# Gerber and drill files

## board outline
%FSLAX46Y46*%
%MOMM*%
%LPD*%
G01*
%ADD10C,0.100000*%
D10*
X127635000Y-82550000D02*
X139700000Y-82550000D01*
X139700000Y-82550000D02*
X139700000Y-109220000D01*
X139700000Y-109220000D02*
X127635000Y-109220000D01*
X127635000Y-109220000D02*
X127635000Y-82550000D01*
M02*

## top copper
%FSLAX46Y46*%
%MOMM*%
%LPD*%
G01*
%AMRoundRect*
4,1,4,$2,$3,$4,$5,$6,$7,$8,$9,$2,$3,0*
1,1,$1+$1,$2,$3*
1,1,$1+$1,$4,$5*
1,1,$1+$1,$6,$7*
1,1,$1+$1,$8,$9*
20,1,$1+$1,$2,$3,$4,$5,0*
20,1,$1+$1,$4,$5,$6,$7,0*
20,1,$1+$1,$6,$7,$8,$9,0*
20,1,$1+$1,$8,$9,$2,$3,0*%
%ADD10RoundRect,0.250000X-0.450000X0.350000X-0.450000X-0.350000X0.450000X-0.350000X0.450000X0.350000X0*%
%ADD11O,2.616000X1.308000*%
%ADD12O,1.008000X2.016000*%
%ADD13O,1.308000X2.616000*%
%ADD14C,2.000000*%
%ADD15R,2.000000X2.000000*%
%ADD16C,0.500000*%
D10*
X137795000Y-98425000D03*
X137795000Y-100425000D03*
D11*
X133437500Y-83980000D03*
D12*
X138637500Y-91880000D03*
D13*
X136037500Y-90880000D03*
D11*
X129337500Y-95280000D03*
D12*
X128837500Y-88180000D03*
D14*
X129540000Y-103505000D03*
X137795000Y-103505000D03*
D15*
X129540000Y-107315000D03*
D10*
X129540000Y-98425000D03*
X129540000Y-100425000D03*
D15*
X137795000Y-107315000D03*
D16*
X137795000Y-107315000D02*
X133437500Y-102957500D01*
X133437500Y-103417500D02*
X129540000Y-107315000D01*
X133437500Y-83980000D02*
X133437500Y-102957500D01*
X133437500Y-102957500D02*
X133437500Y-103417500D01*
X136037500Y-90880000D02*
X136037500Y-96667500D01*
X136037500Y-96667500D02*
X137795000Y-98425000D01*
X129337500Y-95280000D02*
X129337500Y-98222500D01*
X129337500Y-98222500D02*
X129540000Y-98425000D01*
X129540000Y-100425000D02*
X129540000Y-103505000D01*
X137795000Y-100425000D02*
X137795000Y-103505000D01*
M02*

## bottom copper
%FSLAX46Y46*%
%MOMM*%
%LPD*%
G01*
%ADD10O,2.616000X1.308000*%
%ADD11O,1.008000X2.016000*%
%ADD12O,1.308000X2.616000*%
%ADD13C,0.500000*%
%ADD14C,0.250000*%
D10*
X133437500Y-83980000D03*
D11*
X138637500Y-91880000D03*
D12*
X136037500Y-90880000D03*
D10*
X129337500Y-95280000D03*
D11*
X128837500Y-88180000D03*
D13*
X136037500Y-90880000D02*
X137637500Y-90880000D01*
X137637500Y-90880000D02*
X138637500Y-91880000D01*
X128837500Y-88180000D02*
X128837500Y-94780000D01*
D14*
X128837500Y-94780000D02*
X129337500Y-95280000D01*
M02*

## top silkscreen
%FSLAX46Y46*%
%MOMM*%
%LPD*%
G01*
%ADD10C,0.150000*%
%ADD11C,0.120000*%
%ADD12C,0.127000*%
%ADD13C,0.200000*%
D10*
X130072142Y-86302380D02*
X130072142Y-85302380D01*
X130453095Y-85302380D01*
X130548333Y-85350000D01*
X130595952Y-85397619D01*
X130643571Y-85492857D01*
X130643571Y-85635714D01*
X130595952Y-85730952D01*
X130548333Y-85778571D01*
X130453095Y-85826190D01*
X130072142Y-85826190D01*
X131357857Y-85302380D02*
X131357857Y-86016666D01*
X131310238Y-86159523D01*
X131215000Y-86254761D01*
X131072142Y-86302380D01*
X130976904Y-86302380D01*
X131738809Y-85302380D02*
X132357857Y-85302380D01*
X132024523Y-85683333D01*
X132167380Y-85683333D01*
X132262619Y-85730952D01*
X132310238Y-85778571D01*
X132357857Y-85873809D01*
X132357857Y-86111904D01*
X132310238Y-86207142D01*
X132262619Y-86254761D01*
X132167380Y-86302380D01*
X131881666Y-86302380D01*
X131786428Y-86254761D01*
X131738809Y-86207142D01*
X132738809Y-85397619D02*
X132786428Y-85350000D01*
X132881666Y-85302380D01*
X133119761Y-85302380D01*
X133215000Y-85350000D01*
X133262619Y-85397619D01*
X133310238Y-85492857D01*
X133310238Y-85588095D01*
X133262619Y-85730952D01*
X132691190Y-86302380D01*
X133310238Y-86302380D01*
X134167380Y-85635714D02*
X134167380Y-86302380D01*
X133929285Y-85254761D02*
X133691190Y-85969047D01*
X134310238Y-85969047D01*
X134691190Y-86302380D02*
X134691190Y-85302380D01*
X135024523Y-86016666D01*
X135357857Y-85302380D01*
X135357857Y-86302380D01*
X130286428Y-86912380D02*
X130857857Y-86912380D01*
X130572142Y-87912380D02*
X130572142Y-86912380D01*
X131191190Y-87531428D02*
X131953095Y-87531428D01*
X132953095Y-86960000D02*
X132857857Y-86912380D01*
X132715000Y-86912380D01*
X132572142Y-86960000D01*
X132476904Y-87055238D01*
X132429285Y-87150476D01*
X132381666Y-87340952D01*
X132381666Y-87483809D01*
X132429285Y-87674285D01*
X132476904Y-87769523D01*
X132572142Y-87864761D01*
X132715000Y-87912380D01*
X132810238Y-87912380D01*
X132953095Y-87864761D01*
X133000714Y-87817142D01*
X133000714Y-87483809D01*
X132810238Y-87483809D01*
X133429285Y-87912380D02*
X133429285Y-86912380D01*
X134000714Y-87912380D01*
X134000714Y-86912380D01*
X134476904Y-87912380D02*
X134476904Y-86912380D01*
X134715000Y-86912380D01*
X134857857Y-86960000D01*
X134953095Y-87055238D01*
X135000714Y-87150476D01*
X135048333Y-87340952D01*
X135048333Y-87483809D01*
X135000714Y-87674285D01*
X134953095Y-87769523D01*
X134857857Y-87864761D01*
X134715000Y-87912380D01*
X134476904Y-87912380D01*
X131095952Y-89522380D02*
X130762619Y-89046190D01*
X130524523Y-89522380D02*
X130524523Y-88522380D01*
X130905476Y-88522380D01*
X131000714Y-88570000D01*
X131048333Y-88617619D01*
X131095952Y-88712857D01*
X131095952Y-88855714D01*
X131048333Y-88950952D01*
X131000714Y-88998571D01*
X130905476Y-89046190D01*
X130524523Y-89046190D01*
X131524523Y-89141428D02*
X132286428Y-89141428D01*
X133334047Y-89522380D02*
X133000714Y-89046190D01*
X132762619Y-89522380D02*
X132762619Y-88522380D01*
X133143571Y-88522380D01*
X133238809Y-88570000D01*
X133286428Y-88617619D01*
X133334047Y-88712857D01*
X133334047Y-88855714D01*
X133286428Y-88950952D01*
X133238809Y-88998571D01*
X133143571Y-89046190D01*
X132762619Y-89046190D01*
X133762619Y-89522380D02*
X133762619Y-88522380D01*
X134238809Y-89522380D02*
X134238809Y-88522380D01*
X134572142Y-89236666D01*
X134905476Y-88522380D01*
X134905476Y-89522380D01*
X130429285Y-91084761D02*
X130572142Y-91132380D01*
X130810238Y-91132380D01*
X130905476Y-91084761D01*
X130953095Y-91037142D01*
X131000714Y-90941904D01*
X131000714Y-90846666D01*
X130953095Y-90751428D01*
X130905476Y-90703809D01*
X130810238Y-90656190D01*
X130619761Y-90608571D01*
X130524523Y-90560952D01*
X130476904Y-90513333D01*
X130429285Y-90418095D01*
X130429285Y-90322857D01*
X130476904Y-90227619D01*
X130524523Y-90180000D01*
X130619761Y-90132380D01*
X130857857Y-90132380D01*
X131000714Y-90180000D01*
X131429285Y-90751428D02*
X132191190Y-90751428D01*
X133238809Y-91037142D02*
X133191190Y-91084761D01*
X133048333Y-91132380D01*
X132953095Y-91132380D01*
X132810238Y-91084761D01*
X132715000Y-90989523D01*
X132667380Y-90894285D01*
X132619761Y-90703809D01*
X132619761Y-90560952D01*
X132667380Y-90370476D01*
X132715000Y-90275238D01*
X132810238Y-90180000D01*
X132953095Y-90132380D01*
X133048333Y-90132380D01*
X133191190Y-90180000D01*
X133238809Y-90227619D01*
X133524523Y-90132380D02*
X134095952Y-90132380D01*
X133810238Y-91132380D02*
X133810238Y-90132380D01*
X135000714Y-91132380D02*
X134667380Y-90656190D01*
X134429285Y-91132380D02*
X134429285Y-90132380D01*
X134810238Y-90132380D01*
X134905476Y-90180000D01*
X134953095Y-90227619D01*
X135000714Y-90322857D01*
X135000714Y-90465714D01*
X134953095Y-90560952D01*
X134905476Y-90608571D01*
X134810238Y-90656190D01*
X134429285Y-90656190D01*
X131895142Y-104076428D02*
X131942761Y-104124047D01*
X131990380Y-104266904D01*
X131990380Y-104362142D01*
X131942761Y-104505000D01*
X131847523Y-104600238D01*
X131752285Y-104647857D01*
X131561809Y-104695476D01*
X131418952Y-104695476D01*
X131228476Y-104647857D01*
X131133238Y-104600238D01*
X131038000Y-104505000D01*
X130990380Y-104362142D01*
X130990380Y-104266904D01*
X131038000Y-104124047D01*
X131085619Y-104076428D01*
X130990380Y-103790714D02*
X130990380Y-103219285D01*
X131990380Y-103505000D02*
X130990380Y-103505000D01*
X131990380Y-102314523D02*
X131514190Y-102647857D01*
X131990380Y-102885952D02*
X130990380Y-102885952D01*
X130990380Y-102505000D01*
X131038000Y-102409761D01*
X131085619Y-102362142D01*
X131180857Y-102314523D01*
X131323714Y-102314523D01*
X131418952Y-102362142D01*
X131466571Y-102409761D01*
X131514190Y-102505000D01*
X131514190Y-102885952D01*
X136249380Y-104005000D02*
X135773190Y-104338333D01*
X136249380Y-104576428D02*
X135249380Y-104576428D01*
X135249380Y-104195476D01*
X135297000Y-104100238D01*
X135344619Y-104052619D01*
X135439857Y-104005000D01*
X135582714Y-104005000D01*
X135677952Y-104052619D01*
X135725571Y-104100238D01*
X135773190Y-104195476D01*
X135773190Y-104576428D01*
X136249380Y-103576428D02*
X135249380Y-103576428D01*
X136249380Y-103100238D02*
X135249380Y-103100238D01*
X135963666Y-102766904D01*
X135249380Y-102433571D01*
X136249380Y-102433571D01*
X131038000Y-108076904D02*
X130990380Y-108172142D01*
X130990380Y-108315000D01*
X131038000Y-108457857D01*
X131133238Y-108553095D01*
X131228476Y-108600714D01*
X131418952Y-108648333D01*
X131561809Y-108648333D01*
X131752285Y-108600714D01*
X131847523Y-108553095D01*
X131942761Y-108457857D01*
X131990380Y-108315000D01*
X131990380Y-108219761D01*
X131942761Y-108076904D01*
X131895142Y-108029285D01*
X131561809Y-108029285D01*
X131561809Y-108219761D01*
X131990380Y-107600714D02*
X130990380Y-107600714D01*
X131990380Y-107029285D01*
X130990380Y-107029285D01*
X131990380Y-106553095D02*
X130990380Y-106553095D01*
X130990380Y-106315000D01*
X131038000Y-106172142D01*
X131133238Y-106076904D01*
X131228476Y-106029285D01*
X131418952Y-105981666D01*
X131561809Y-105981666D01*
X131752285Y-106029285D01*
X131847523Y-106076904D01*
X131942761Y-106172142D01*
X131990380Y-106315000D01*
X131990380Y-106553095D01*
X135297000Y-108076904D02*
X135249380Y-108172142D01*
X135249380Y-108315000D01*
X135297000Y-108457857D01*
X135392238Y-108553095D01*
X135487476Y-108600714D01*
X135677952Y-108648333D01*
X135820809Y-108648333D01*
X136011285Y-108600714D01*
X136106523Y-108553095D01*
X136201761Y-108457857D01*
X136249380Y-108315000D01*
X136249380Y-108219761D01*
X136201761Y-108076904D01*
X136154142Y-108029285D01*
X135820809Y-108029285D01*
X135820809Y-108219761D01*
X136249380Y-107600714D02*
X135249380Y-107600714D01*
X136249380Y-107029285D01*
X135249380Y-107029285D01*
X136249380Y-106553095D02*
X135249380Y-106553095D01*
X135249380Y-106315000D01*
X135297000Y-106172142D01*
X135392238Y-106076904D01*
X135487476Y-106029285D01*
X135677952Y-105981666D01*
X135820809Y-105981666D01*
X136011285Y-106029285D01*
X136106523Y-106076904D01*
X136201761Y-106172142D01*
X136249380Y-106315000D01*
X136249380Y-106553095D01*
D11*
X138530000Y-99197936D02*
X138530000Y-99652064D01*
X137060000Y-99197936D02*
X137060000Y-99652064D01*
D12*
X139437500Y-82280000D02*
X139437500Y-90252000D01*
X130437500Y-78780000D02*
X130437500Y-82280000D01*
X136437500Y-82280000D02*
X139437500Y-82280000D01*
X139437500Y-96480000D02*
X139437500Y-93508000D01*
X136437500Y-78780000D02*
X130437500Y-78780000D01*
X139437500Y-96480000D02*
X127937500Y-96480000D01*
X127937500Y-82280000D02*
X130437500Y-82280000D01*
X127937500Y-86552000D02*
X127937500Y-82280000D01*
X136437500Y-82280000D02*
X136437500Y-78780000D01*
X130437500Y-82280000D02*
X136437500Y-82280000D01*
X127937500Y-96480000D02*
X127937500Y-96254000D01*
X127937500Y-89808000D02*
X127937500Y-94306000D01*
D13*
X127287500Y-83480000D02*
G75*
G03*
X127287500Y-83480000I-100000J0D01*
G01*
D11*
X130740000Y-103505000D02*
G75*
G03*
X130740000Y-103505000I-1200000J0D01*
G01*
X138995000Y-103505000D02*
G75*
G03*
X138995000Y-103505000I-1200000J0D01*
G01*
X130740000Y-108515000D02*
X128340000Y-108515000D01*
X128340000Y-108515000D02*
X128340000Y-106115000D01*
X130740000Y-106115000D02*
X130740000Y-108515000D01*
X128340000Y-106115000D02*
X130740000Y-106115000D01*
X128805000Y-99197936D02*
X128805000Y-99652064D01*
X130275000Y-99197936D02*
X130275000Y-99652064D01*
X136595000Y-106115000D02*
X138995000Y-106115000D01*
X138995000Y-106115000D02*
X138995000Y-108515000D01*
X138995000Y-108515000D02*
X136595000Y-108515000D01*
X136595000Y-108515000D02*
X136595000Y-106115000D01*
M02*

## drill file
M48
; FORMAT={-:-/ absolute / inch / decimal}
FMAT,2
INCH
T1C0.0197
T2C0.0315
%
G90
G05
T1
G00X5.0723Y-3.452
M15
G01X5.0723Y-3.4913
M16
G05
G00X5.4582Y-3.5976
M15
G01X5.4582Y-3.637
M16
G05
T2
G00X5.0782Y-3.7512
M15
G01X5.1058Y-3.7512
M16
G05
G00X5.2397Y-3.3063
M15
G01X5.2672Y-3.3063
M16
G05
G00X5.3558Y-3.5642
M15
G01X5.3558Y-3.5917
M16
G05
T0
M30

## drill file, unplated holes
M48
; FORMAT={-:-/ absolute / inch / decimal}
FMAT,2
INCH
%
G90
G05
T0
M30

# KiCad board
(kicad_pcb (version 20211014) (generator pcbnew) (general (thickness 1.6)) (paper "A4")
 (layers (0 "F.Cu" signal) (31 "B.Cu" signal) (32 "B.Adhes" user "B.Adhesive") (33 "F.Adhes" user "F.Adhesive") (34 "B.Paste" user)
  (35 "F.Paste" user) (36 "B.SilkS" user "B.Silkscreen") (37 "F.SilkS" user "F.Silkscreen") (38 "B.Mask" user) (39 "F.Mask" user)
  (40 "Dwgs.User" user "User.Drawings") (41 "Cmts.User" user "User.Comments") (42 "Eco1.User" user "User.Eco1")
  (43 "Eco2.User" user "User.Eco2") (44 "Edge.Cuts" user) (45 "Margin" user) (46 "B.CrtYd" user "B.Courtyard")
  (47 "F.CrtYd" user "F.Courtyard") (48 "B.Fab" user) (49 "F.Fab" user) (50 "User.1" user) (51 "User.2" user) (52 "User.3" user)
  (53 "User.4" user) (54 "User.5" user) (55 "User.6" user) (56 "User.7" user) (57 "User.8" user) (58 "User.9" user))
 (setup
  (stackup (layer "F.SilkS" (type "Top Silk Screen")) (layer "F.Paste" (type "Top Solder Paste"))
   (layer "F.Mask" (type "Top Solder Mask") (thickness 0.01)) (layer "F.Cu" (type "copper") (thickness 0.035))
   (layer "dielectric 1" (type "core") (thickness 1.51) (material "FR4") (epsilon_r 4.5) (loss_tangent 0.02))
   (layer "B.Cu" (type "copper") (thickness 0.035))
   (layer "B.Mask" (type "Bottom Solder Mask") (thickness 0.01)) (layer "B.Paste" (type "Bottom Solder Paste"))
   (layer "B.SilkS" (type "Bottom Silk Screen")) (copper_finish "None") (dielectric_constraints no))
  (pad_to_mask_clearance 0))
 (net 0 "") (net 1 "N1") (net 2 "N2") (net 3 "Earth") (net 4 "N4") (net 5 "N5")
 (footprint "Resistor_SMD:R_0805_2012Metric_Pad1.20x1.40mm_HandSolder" (layer "F.Cu") (at 137.795 99.425 -90)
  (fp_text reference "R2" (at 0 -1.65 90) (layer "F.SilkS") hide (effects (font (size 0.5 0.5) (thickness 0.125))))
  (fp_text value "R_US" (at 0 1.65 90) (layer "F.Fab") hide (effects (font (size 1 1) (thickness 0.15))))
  (fp_line (start -0.227064 -0.735) (end 0.227064 -0.735) (layer "F.SilkS") (width 0.12))
  (fp_line (start -0.227064 0.735) (end 0.227064 0.735) (layer "F.SilkS") (width 0.12))
  (pad "1" smd roundrect (at -1 0 270) (size 1.2 1.4) (layers "F.Cu" "F.Paste" "F.Mask") (roundrect_rratio 0.2083333333) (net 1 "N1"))
  (pad "2" smd roundrect (at 1 0 270) (size 1.2 1.4) (layers "F.Cu" "F.Paste" "F.Mask") (roundrect_rratio 0.2083333333) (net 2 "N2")))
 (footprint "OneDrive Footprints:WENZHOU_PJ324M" (layer "F.Cu") (at 133.4375 89.38)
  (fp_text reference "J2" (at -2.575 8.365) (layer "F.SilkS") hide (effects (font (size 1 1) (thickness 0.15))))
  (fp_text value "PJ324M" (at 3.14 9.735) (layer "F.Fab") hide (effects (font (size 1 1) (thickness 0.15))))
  (fp_line (start 6 -7.1) (end 6 0.872) (layer "F.SilkS") (width 0.127))
  (fp_line (start -3 -10.6) (end -3 -7.1) (layer "F.SilkS") (width 0.127))
  (fp_line (start 3 -7.1) (end 6 -7.1) (layer "F.SilkS") (width 0.127))
  (fp_line (start 6 7.1) (end 6 4.128) (layer "F.SilkS") (width 0.127))
  (fp_line (start 3 -10.6) (end -3 -10.6) (layer "F.SilkS") (width 0.127))
  (fp_line (start 6 7.1) (end -5.5 7.1) (layer "F.SilkS") (width 0.127))
  (fp_line (start -5.5 -7.1) (end -3 -7.1) (layer "F.SilkS") (width 0.127))
  (fp_line (start -5.5 -2.828) (end -5.5 -7.1) (layer "F.SilkS") (width 0.127))
  (fp_line (start 3 -7.1) (end 3 -10.6) (layer "F.SilkS") (width 0.127))
  (fp_line (start -3 -7.1) (end 3 -7.1) (layer "F.SilkS") (width 0.127))
  (fp_line (start -5.5 7.1) (end -5.5 6.874) (layer "F.SilkS") (width 0.127))
  (fp_line (start -5.5 0.428) (end -5.5 4.926) (layer "F.SilkS") (width 0.127))
  (fp_circle (center -6.25 -5.9) (end -6.15 -5.9) (layer "F.SilkS") (width 0.2) (fill none))
  (pad "1" thru_hole oval locked (at 0 -5.4) (size 2.616 1.308) (drill oval 1.5 0.8) (layers *.Cu *.Mask) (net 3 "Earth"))
  (pad "2" thru_hole oval locked (at 5.2 2.5) (size 1.008 2.016) (drill oval 0.5 1.5) (layers *.Cu *.Mask) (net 1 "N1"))
  (pad "3" thru_hole oval locked (at 2.6 1.5) (size 1.308 2.616) (drill oval 0.8 1.5) (layers *.Cu *.Mask) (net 1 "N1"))
  (pad "4" thru_hole oval locked (at -4.1 5.9) (size 2.616 1.308) (drill oval 1.5 0.8) (layers *.Cu *.Mask) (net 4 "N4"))
  (pad "5" thru_hole oval locked (at -4.6 -1.2) (size 1.008 2.016) (drill oval 0.5 1.5) (layers *.Cu *.Mask) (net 4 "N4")))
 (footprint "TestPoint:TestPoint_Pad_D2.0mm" (layer "F.Cu") (at 129.54 103.505 -90)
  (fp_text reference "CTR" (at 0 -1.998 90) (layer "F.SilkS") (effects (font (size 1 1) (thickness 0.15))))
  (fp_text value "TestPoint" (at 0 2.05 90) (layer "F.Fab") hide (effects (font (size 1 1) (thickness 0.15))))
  (fp_circle (center 0 0) (end 0 1.2) (layer "F.SilkS") (width 0.12) (fill none))
  (pad "1" smd circle (at 0 0 270) (size 2 2) (layers "F.Cu" "F.Mask") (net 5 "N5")))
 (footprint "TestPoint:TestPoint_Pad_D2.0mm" (layer "F.Cu") (at 137.795 103.505 90)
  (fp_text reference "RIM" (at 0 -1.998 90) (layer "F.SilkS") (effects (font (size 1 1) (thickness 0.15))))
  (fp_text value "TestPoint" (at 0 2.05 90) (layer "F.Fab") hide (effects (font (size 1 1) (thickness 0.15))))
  (fp_circle (center 0 0) (end 0 1.2) (layer "F.SilkS") (width 0.12) (fill none))
  (pad "1" smd circle (at 0 0 90) (size 2 2) (layers "F.Cu" "F.Mask") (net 2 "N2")))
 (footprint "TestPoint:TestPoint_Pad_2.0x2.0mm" (layer "F.Cu") (at 129.54 107.315 -90)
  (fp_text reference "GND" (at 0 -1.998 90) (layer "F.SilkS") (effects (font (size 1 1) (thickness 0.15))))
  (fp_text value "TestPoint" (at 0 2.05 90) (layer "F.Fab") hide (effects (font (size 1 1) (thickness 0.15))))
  (fp_line (start 1.2 -1.2) (end 1.2 1.2) (layer "F.SilkS") (width 0.12))
  (fp_line (start 1.2 1.2) (end -1.2 1.2) (layer "F.SilkS") (width 0.12))
  (fp_line (start -1.2 -1.2) (end 1.2 -1.2) (layer "F.SilkS") (width 0.12))
  (fp_line (start -1.2 1.2) (end -1.2 -1.2) (layer "F.SilkS") (width 0.12))
  (pad "1" smd rect (at 0 0 270) (size 2 2) (layers "F.Cu" "F.Mask") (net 3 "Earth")))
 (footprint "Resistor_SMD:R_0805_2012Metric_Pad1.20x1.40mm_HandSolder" (layer "F.Cu") (at 129.54 99.425 -90)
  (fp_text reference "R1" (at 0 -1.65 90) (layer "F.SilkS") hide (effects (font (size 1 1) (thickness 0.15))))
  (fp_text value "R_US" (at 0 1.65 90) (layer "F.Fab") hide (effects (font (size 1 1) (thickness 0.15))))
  (fp_line (start -0.227064 0.735) (end 0.227064 0.735) (layer "F.SilkS") (width 0.12))
  (fp_line (start -0.227064 -0.735) (end 0.227064 -0.735) (layer "F.SilkS") (width 0.12))
  (pad "1" smd roundrect (at -1 0 270) (size 1.2 1.4) (layers "F.Cu" "F.Paste" "F.Mask") (roundrect_rratio 0.2083333333) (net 4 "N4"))
  (pad "2" smd roundrect (at 1 0 270) (size 1.2 1.4) (layers "F.Cu" "F.Paste" "F.Mask") (roundrect_rratio 0.2083333333) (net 5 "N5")))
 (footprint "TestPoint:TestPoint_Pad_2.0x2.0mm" (layer "F.Cu") (at 137.795 107.315 90)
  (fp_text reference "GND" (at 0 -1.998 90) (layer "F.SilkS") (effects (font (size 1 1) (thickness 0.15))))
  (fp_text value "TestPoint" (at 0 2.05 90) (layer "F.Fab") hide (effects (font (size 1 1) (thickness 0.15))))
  (fp_line (start 1.2 -1.2) (end 1.2 1.2) (layer "F.SilkS") (width 0.12))
  (fp_line (start 1.2 1.2) (end -1.2 1.2) (layer "F.SilkS") (width 0.12))
  (fp_line (start -1.2 1.2) (end -1.2 -1.2) (layer "F.SilkS") (width 0.12))
  (fp_line (start -1.2 -1.2) (end 1.2 -1.2) (layer "F.SilkS") (width 0.12))
  (pad "1" smd rect (at 0 0 90) (size 2 2) (layers "F.Cu" "F.Mask") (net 3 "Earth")))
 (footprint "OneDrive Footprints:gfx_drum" (layer "B.Cu") (at 133.35 88.265 -90)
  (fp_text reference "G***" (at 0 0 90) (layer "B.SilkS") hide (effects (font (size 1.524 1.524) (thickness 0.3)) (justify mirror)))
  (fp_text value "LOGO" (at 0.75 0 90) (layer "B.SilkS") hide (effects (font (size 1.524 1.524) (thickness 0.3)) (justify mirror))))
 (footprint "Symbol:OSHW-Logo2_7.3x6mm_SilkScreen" (layer "B.Cu") (at 132.08 100.965 -90)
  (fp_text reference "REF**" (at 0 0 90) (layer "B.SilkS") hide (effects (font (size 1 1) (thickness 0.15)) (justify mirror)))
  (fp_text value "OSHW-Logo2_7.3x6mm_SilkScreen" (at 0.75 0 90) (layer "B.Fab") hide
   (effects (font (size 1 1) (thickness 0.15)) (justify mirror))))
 (gr_rect (start 127.635 82.55) (end 139.7 109.22) (layer "Edge.Cuts") (width 0.1) (fill none))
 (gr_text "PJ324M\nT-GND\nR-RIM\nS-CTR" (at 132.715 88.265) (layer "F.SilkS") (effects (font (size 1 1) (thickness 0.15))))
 (segment (start 137.795 107.315) (end 133.4375 102.9575) (width 0.5) (layer "F.Cu") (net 3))
 (segment (start 133.4375 103.4175) (end 129.54 107.315) (width 0.5) (layer "F.Cu") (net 3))
 (segment (start 133.4375 83.98) (end 133.4375 102.9575) (width 0.5) (layer "F.Cu") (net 3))
 (segment (start 133.4375 102.9575) (end 133.4375 103.4175) (width 0.5) (layer "F.Cu") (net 3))
 (segment (start 136.0375 90.88) (end 136.0375 96.6675) (width 0.5) (layer "F.Cu") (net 1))
 (segment (start 136.0375 96.6675) (end 137.795 98.425) (width 0.5) (layer "F.Cu") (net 1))
 (segment (start 136.0375 90.88) (end 137.6375 90.88) (width 0.5) (layer "B.Cu") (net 1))
 (segment (start 137.6375 90.88) (end 138.6375 91.88) (width 0.5) (layer "B.Cu") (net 1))
 (segment (start 129.3375 95.28) (end 129.3375 98.2225) (width 0.5) (layer "F.Cu") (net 4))
 (segment (start 129.3375 98.2225) (end 129.54 98.425) (width 0.5) (layer "F.Cu") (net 4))
 (segment (start 128.8375 88.18) (end 128.8375 94.78) (width 0.5) (layer "B.Cu") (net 4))
 (segment (start 128.8375 94.78) (end 129.3375 95.28) (width 0.25) (layer "B.Cu") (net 4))
 (segment (start 129.54 100.425) (end 129.54 103.505) (width 0.5) (layer "F.Cu") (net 5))
 (segment (start 137.795 100.425) (end 137.795 103.505) (width 0.5) (layer "F.Cu") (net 2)))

